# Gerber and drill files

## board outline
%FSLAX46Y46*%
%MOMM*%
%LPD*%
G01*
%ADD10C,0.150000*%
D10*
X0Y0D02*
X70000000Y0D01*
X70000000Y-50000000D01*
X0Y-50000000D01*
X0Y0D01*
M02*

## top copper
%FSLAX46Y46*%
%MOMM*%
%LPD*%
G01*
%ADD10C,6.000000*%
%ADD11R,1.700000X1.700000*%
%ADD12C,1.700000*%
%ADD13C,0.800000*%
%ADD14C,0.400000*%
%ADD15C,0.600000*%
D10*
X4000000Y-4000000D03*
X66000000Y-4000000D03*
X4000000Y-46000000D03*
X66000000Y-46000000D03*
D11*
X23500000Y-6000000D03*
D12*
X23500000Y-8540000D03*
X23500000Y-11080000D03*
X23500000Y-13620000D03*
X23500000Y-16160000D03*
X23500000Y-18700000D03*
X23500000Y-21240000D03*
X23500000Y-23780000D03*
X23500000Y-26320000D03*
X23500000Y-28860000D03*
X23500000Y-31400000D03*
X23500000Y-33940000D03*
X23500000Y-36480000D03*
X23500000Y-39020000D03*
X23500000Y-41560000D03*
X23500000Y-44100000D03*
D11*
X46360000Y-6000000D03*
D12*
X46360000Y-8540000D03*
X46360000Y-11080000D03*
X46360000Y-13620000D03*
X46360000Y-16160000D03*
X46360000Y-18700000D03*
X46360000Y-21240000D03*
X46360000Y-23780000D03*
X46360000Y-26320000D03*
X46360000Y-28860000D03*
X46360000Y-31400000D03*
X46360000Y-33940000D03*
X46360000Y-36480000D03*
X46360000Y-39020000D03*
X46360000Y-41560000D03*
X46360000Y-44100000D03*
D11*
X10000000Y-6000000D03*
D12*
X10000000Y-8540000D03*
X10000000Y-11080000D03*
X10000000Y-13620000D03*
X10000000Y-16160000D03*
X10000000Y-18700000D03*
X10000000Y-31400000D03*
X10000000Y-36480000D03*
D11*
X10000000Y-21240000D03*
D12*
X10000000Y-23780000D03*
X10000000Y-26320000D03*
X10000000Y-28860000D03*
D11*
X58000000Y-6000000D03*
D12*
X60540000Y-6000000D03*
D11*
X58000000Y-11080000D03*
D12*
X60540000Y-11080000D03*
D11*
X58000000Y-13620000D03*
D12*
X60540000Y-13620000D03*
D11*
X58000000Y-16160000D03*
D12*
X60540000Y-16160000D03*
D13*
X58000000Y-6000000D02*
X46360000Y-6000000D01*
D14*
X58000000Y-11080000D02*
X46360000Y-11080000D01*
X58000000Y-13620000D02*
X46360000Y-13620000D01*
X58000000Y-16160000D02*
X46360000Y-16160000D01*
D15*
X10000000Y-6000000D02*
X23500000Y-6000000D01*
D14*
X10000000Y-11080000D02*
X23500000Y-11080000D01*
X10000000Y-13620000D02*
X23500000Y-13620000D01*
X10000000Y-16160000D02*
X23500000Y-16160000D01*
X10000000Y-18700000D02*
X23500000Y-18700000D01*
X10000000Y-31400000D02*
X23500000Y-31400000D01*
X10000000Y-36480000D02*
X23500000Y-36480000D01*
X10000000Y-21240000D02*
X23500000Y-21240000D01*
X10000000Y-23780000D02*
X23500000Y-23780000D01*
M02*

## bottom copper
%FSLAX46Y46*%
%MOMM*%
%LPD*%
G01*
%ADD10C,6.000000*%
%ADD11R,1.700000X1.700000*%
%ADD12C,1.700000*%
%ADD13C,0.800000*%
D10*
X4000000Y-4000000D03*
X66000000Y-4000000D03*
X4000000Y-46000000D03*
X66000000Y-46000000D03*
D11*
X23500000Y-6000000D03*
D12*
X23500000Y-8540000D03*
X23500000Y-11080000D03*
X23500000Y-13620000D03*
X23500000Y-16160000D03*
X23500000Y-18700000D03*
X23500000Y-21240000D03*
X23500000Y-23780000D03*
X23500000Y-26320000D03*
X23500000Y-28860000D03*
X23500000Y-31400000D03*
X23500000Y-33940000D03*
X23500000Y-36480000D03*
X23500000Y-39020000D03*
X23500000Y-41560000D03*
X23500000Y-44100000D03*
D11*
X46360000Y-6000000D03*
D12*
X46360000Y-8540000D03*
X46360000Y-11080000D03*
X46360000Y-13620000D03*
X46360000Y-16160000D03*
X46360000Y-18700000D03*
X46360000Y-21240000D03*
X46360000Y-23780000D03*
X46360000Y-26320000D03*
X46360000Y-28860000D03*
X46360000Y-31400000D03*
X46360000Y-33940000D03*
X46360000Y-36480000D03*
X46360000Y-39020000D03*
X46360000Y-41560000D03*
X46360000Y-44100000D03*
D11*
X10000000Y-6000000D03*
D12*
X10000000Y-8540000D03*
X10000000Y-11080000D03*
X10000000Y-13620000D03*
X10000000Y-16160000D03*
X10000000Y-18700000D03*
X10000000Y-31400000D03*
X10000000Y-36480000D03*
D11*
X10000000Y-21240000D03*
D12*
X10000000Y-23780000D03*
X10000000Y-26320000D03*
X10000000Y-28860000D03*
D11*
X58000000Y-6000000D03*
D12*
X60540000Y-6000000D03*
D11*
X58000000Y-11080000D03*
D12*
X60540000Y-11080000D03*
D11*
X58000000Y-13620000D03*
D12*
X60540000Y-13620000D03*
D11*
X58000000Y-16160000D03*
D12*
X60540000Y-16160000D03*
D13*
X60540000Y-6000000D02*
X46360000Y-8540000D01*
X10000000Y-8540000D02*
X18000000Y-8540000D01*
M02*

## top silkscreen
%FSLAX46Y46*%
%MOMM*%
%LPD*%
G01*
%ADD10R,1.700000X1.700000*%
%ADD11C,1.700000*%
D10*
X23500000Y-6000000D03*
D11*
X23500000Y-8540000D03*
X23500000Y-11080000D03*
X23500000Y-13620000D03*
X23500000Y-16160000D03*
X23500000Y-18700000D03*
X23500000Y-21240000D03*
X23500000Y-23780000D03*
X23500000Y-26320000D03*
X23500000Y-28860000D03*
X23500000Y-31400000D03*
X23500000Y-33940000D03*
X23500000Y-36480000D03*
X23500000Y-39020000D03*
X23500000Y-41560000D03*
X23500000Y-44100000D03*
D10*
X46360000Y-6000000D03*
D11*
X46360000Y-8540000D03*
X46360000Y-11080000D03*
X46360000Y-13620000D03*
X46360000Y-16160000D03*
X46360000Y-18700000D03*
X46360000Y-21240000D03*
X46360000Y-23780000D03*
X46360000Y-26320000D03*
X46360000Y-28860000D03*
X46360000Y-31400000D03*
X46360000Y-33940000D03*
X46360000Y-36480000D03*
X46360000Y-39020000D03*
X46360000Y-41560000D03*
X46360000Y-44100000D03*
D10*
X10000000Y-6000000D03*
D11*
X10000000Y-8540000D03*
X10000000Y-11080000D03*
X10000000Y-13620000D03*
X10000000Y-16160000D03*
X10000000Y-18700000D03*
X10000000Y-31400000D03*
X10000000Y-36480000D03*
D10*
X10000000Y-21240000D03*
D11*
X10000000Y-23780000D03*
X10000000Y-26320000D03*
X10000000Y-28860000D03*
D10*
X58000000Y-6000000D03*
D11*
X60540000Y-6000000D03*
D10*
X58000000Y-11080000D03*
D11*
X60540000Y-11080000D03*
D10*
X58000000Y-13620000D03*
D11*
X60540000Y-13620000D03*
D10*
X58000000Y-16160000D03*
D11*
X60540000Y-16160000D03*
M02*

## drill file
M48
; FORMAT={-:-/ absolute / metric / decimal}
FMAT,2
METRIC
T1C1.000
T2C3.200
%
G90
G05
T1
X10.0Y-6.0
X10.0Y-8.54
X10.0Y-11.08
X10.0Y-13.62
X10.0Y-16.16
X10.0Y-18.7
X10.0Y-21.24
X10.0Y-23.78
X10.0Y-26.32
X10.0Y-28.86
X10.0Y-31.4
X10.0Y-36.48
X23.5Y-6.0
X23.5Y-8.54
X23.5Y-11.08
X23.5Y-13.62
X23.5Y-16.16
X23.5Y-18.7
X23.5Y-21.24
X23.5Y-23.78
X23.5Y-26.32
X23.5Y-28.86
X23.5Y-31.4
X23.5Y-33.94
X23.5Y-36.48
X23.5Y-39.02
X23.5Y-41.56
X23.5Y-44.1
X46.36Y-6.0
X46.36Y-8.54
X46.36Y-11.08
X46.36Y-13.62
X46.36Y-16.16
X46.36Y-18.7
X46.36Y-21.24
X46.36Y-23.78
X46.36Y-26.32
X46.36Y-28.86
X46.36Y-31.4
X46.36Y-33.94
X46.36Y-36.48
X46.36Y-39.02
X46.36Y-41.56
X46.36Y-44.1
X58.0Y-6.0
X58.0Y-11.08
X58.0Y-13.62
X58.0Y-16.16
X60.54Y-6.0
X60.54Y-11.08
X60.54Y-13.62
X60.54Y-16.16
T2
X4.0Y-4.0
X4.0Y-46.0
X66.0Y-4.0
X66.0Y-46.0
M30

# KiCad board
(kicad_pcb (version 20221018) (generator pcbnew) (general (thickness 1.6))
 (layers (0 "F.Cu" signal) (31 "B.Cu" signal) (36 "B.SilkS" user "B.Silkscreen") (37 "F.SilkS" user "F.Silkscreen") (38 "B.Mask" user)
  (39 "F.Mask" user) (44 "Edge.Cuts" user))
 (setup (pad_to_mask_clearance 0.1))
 (gr_rect (start 0 0) (end 70.0 50.0) (layer "Edge.Cuts") (width 0.15) (fill none))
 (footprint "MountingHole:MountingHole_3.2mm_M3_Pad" (layer "F.Cu") (at 4.0 4.0)
  (pad "" np_thru_hole circle (at 0 0) (size 6.0 6.0) (drill 3.2) (layers *.Cu *.Mask)))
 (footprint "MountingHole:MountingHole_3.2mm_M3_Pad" (layer "F.Cu") (at 66.0 4.0)
  (pad "" np_thru_hole circle (at 0 0) (size 6.0 6.0) (drill 3.2) (layers *.Cu *.Mask)))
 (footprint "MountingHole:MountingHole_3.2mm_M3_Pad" (layer "F.Cu") (at 4.0 46.0)
  (pad "" np_thru_hole circle (at 0 0) (size 6.0 6.0) (drill 3.2) (layers *.Cu *.Mask)))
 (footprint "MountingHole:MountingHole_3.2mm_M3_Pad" (layer "F.Cu") (at 66.0 46.0)
  (pad "" np_thru_hole circle (at 0 0) (size 6.0 6.0) (drill 3.2) (layers *.Cu *.Mask)))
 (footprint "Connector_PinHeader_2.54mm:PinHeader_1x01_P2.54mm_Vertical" (layer "F.Cu") (at 23.5 6.0)
  (pad "1" thru_hole rect (at 0 0) (size 1.7 1.7) (drill 1.0) (layers *.Cu *.Mask "F.SilkS")))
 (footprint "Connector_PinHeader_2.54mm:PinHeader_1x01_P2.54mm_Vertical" (layer "F.Cu") (at 23.5 8.54)
  (pad "1" thru_hole circle (at 0 0) (size 1.7 1.7) (drill 1.0) (layers *.Cu *.Mask "F.SilkS")))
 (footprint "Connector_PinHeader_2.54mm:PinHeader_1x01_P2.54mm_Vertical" (layer "F.Cu") (at 23.5 11.08)
  (pad "1" thru_hole circle (at 0 0) (size 1.7 1.7) (drill 1.0) (layers *.Cu *.Mask "F.SilkS")))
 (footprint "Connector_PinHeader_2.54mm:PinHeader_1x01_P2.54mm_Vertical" (layer "F.Cu") (at 23.5 13.620000000000001)
  (pad "1" thru_hole circle (at 0 0) (size 1.7 1.7) (drill 1.0) (layers *.Cu *.Mask "F.SilkS")))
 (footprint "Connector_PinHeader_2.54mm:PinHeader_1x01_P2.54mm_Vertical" (layer "F.Cu") (at 23.5 16.16)
  (pad "1" thru_hole circle (at 0 0) (size 1.7 1.7) (drill 1.0) (layers *.Cu *.Mask "F.SilkS")))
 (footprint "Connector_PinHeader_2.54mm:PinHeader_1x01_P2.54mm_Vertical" (layer "F.Cu") (at 23.5 18.7)
  (pad "1" thru_hole circle (at 0 0) (size 1.7 1.7) (drill 1.0) (layers *.Cu *.Mask "F.SilkS")))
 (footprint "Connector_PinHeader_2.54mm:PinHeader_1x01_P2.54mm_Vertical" (layer "F.Cu") (at 23.5 21.240000000000002)
  (pad "1" thru_hole circle (at 0 0) (size 1.7 1.7) (drill 1.0) (layers *.Cu *.Mask "F.SilkS")))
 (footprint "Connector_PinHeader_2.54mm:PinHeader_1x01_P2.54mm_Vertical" (layer "F.Cu") (at 23.5 23.78)
  (pad "1" thru_hole circle (at 0 0) (size 1.7 1.7) (drill 1.0) (layers *.Cu *.Mask "F.SilkS")))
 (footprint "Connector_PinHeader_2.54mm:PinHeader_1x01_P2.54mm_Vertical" (layer "F.Cu") (at 23.5 26.32)
  (pad "1" thru_hole circle (at 0 0) (size 1.7 1.7) (drill 1.0) (layers *.Cu *.Mask "F.SilkS")))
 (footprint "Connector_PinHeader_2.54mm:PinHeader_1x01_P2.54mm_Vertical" (layer "F.Cu") (at 23.5 28.86)
  (pad "1" thru_hole circle (at 0 0) (size 1.7 1.7) (drill 1.0) (layers *.Cu *.Mask "F.SilkS")))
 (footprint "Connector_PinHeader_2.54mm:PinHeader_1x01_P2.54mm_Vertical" (layer "F.Cu") (at 23.5 31.4)
  (pad "1" thru_hole circle (at 0 0) (size 1.7 1.7) (drill 1.0) (layers *.Cu *.Mask "F.SilkS")))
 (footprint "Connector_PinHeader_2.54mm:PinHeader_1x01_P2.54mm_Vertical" (layer "F.Cu") (at 23.5 33.94)
  (pad "1" thru_hole circle (at 0 0) (size 1.7 1.7) (drill 1.0) (layers *.Cu *.Mask "F.SilkS")))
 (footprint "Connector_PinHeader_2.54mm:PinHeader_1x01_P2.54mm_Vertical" (layer "F.Cu") (at 23.5 36.480000000000004)
  (pad "1" thru_hole circle (at 0 0) (size 1.7 1.7) (drill 1.0) (layers *.Cu *.Mask "F.SilkS")))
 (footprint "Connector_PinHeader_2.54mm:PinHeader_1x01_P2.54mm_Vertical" (layer "F.Cu") (at 23.5 39.02)
  (pad "1" thru_hole circle (at 0 0) (size 1.7 1.7) (drill 1.0) (layers *.Cu *.Mask "F.SilkS")))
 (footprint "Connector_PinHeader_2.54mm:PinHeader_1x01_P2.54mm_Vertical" (layer "F.Cu") (at 23.5 41.56)
  (pad "1" thru_hole circle (at 0 0) (size 1.7 1.7) (drill 1.0) (layers *.Cu *.Mask "F.SilkS")))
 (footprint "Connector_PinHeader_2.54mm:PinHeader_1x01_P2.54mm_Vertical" (layer "F.Cu") (at 23.5 44.1)
  (pad "1" thru_hole circle (at 0 0) (size 1.7 1.7) (drill 1.0) (layers *.Cu *.Mask "F.SilkS")))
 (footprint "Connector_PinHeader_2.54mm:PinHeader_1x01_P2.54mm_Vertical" (layer "F.Cu") (at 46.36 6.0)
  (pad "1" thru_hole rect (at 0 0) (size 1.7 1.7) (drill 1.0) (layers *.Cu *.Mask "F.SilkS")))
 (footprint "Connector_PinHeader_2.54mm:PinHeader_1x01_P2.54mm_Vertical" (layer "F.Cu") (at 46.36 8.54)
  (pad "1" thru_hole circle (at 0 0) (size 1.7 1.7) (drill 1.0) (layers *.Cu *.Mask "F.SilkS")))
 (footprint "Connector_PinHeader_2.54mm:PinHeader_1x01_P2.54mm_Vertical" (layer "F.Cu") (at 46.36 11.08)
  (pad "1" thru_hole circle (at 0 0) (size 1.7 1.7) (drill 1.0) (layers *.Cu *.Mask "F.SilkS")))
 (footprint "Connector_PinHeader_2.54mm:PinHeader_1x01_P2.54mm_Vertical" (layer "F.Cu") (at 46.36 13.620000000000001)
  (pad "1" thru_hole circle (at 0 0) (size 1.7 1.7) (drill 1.0) (layers *.Cu *.Mask "F.SilkS")))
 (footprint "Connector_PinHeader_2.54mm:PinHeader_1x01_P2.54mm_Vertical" (layer "F.Cu") (at 46.36 16.16)
  (pad "1" thru_hole circle (at 0 0) (size 1.7 1.7) (drill 1.0) (layers *.Cu *.Mask "F.SilkS")))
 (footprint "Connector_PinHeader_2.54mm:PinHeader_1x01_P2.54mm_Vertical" (layer "F.Cu") (at 46.36 18.7)
  (pad "1" thru_hole circle (at 0 0) (size 1.7 1.7) (drill 1.0) (layers *.Cu *.Mask "F.SilkS")))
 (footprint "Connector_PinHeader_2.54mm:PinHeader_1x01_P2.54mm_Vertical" (layer "F.Cu") (at 46.36 21.240000000000002)
  (pad "1" thru_hole circle (at 0 0) (size 1.7 1.7) (drill 1.0) (layers *.Cu *.Mask "F.SilkS")))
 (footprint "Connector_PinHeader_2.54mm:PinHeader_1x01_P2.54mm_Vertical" (layer "F.Cu") (at 46.36 23.78)
  (pad "1" thru_hole circle (at 0 0) (size 1.7 1.7) (drill 1.0) (layers *.Cu *.Mask "F.SilkS")))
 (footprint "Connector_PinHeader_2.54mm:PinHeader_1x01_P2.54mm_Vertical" (layer "F.Cu") (at 46.36 26.32)
  (pad "1" thru_hole circle (at 0 0) (size 1.7 1.7) (drill 1.0) (layers *.Cu *.Mask "F.SilkS")))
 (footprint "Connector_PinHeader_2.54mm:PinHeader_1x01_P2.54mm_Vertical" (layer "F.Cu") (at 46.36 28.86)
  (pad "1" thru_hole circle (at 0 0) (size 1.7 1.7) (drill 1.0) (layers *.Cu *.Mask "F.SilkS")))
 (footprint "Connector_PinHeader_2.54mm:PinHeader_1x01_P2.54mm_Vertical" (layer "F.Cu") (at 46.36 31.4)
  (pad "1" thru_hole circle (at 0 0) (size 1.7 1.7) (drill 1.0) (layers *.Cu *.Mask "F.SilkS")))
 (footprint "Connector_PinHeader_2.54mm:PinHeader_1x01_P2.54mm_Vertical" (layer "F.Cu") (at 46.36 33.94)
  (pad "1" thru_hole circle (at 0 0) (size 1.7 1.7) (drill 1.0) (layers *.Cu *.Mask "F.SilkS")))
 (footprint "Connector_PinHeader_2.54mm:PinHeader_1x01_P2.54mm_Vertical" (layer "F.Cu") (at 46.36 36.480000000000004)
  (pad "1" thru_hole circle (at 0 0) (size 1.7 1.7) (drill 1.0) (layers *.Cu *.Mask "F.SilkS")))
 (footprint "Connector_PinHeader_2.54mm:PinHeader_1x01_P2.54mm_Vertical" (layer "F.Cu") (at 46.36 39.02)
  (pad "1" thru_hole circle (at 0 0) (size 1.7 1.7) (drill 1.0) (layers *.Cu *.Mask "F.SilkS")))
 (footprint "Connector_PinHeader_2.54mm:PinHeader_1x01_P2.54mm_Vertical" (layer "F.Cu") (at 46.36 41.56)
  (pad "1" thru_hole circle (at 0 0) (size 1.7 1.7) (drill 1.0) (layers *.Cu *.Mask "F.SilkS")))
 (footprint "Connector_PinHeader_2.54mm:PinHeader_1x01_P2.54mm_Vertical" (layer "F.Cu") (at 46.36 44.1)
  (pad "1" thru_hole circle (at 0 0) (size 1.7 1.7) (drill 1.0) (layers *.Cu *.Mask "F.SilkS")))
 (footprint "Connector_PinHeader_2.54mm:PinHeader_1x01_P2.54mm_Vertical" (layer "F.Cu") (at 10.0 6.0)
  (pad "1" thru_hole rect (at 0 0) (size 1.7 1.7) (drill 1.0) (layers *.Cu *.Mask "F.SilkS")))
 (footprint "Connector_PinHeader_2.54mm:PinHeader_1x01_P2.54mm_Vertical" (layer "F.Cu") (at 10.0 8.54)
  (pad "1" thru_hole circle (at 0 0) (size 1.7 1.7) (drill 1.0) (layers *.Cu *.Mask "F.SilkS")))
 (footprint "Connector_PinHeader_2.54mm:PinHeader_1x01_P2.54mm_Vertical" (layer "F.Cu") (at 10.0 11.08)
  (pad "1" thru_hole circle (at 0 0) (size 1.7 1.7) (drill 1.0) (layers *.Cu *.Mask "F.SilkS")))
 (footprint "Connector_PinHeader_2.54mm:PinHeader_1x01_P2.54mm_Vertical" (layer "F.Cu") (at 10.0 13.62)
  (pad "1" thru_hole circle (at 0 0) (size 1.7 1.7) (drill 1.0) (layers *.Cu *.Mask "F.SilkS")))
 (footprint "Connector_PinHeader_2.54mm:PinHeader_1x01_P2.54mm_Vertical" (layer "F.Cu") (at 10.0 16.16)
  (pad "1" thru_hole circle (at 0 0) (size 1.7 1.7) (drill 1.0) (layers *.Cu *.Mask "F.SilkS")))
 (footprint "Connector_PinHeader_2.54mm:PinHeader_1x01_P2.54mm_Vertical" (layer "F.Cu") (at 10.0 18.7)
  (pad "1" thru_hole circle (at 0 0) (size 1.7 1.7) (drill 1.0) (layers *.Cu *.Mask "F.SilkS")))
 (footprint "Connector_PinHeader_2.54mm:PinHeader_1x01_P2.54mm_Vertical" (layer "F.Cu") (at 10.0 31.4)
  (pad "1" thru_hole circle (at 0 0) (size 1.7 1.7) (drill 1.0) (layers *.Cu *.Mask "F.SilkS")))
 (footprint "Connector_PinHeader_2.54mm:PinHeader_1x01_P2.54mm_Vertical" (layer "F.Cu") (at 10.0 36.48)
  (pad "1" thru_hole circle (at 0 0) (size 1.7 1.7) (drill 1.0) (layers *.Cu *.Mask "F.SilkS")))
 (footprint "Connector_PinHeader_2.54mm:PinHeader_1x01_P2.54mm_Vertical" (layer "F.Cu") (at 10.0 21.24)
  (pad "1" thru_hole rect (at 0 0) (size 1.7 1.7) (drill 1.0) (layers *.Cu *.Mask "F.SilkS")))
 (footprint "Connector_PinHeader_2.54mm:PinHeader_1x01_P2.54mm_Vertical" (layer "F.Cu") (at 10.0 23.779999999999998)
  (pad "1" thru_hole circle (at 0 0) (size 1.7 1.7) (drill 1.0) (layers *.Cu *.Mask "F.SilkS")))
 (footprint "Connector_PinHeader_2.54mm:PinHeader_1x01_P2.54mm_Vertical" (layer "F.Cu") (at 10.0 26.32)
  (pad "1" thru_hole circle (at 0 0) (size 1.7 1.7) (drill 1.0) (layers *.Cu *.Mask "F.SilkS")))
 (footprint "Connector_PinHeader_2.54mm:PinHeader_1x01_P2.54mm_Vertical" (layer "F.Cu") (at 10.0 28.86)
  (pad "1" thru_hole circle (at 0 0) (size 1.7 1.7) (drill 1.0) (layers *.Cu *.Mask "F.SilkS")))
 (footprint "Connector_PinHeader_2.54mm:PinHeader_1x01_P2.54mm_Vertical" (layer "F.Cu") (at 58.0 6.0)
  (pad "1" thru_hole rect (at 0 0) (size 1.7 1.7) (drill 1.0) (layers *.Cu *.Mask "F.SilkS")))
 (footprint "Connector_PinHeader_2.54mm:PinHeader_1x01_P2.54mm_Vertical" (layer "F.Cu") (at 60.54 6.0)
  (pad "1" thru_hole circle (at 0 0) (size 1.7 1.7) (drill 1.0) (layers *.Cu *.Mask "F.SilkS")))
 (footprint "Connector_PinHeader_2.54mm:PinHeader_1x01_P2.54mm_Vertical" (layer "F.Cu") (at 58.0 11.08)
  (pad "1" thru_hole rect (at 0 0) (size 1.7 1.7) (drill 1.0) (layers *.Cu *.Mask "F.SilkS")))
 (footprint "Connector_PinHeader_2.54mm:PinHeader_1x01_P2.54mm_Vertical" (layer "F.Cu") (at 60.54 11.08)
  (pad "1" thru_hole circle (at 0 0) (size 1.7 1.7) (drill 1.0) (layers *.Cu *.Mask "F.SilkS")))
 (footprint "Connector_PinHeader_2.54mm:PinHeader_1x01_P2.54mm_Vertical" (layer "F.Cu") (at 58.0 13.62)
  (pad "1" thru_hole rect (at 0 0) (size 1.7 1.7) (drill 1.0) (layers *.Cu *.Mask "F.SilkS")))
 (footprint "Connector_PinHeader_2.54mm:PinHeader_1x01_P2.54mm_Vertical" (layer "F.Cu") (at 60.54 13.62)
  (pad "1" thru_hole circle (at 0 0) (size 1.7 1.7) (drill 1.0) (layers *.Cu *.Mask "F.SilkS")))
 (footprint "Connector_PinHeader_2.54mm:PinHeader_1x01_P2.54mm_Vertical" (layer "F.Cu") (at 58.0 16.16)
  (pad "1" thru_hole rect (at 0 0) (size 1.7 1.7) (drill 1.0) (layers *.Cu *.Mask "F.SilkS")))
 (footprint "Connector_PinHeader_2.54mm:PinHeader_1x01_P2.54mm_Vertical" (layer "F.Cu") (at 60.54 16.16)
  (pad "1" thru_hole circle (at 0 0) (size 1.7 1.7) (drill 1.0) (layers *.Cu *.Mask "F.SilkS")))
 (segment (start 58.0 6.0) (end 46.36 6.0) (width 0.8) (layer "F.Cu") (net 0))
 (segment (start 58.0 11.08) (end 46.36 11.08) (width 0.4) (layer "F.Cu") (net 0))
 (segment (start 58.0 13.62) (end 46.36 13.62) (width 0.4) (layer "F.Cu") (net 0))
 (segment (start 58.0 16.16) (end 46.36 16.16) (width 0.4) (layer "F.Cu") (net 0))
 (segment (start 10.0 6.0) (end 23.5 6.0) (width 0.6) (layer "F.Cu") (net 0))
 (segment (start 10.0 11.08) (end 23.5 11.08) (width 0.4) (layer "F.Cu") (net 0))
 (segment (start 10.0 13.62) (end 23.5 13.62) (width 0.4) (layer "F.Cu") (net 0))
 (segment (start 10.0 16.16) (end 23.5 16.16) (width 0.4) (layer "F.Cu") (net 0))
 (segment (start 10.0 18.7) (end 23.5 18.7) (width 0.4) (layer "F.Cu") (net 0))
 (segment (start 10.0 31.4) (end 23.5 31.4) (width 0.4) (layer "F.Cu") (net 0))
 (segment (start 10.0 36.48) (end 23.5 36.48) (width 0.4) (layer "F.Cu") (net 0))
 (segment (start 10.0 21.24) (end 23.5 21.24) (width 0.4) (layer "F.Cu") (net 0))
 (segment (start 10.0 23.78) (end 23.5 23.78) (width 0.4) (layer "F.Cu") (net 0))
 (segment (start 60.54 6.0) (end 46.36 8.54) (width 0.8) (layer "B.Cu") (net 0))
 (segment (start 10.0 8.54) (end 18.0 8.54) (width 0.8) (layer "B.Cu") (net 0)))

